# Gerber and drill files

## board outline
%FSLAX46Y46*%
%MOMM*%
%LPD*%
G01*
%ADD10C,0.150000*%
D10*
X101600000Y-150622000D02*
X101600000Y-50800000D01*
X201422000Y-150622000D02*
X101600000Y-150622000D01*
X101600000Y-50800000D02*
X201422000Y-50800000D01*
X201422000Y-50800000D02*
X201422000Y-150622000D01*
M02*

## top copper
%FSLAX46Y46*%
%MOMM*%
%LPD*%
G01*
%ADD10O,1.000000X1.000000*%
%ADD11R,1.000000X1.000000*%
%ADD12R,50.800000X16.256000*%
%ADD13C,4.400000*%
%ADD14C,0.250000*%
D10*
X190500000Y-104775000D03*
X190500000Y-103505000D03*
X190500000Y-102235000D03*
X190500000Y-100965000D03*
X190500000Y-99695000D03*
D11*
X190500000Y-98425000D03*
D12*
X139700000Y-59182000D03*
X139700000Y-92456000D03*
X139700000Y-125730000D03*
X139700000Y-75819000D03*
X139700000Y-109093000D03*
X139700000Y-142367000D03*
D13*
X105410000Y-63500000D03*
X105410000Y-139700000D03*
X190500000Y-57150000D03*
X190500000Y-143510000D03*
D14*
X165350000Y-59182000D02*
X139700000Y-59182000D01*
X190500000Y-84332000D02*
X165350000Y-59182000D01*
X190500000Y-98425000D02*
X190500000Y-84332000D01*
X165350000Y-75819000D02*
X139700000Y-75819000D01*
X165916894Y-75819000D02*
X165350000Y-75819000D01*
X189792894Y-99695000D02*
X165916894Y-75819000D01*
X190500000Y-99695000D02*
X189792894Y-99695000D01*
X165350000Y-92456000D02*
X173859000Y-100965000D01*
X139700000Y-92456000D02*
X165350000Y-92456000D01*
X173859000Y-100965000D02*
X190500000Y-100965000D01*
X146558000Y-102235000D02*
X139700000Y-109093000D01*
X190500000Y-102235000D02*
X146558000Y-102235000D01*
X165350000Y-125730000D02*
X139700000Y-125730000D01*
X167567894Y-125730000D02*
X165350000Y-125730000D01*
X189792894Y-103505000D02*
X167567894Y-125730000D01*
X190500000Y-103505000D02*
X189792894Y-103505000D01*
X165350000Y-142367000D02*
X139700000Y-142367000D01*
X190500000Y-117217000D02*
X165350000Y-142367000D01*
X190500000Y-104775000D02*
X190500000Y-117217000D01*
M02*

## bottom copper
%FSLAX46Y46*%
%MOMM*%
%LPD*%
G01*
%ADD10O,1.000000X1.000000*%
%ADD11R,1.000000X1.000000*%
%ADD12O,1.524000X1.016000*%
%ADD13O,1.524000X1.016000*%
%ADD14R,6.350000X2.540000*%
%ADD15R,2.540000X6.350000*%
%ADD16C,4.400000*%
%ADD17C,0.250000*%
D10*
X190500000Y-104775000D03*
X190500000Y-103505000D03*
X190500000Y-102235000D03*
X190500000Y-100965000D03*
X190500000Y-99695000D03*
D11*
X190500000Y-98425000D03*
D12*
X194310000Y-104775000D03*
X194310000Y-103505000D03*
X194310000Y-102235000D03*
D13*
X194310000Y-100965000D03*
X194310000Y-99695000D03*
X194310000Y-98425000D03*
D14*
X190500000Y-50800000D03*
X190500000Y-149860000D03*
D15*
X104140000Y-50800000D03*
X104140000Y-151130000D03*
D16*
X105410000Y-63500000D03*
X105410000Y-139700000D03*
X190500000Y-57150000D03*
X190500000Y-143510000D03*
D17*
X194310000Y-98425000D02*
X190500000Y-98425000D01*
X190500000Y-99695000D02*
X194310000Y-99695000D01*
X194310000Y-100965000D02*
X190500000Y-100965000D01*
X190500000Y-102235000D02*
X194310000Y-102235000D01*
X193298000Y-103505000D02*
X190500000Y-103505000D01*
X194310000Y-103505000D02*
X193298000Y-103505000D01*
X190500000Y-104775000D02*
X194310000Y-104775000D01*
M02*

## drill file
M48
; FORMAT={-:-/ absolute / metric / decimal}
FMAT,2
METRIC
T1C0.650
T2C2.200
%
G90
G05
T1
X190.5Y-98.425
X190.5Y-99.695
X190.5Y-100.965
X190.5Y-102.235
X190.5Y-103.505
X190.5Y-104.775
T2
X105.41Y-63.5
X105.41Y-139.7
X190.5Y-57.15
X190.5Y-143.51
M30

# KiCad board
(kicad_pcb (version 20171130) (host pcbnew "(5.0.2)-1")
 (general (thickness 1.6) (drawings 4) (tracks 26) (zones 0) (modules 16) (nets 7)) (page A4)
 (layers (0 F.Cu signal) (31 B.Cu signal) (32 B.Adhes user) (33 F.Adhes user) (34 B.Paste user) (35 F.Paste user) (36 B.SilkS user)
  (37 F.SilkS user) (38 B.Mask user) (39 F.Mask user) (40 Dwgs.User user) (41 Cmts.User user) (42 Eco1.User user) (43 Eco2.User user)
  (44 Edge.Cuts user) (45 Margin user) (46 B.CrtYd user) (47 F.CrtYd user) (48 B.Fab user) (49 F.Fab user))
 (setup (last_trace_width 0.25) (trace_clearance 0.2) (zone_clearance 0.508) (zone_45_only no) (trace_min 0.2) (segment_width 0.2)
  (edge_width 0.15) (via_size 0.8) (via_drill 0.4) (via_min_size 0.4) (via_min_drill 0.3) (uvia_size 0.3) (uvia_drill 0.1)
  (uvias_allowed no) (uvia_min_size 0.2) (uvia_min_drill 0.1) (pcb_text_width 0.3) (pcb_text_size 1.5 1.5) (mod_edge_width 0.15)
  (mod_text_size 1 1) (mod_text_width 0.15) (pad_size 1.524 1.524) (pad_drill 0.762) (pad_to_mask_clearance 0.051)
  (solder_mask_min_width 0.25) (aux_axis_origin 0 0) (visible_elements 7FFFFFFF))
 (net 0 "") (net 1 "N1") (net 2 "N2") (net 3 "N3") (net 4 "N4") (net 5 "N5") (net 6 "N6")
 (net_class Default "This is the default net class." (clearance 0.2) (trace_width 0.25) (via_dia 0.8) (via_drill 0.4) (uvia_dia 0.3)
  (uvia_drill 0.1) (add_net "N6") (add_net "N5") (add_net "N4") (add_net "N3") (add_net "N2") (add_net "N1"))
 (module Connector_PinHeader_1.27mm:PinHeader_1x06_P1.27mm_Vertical (layer F.Cu) (at 190.5 98.425)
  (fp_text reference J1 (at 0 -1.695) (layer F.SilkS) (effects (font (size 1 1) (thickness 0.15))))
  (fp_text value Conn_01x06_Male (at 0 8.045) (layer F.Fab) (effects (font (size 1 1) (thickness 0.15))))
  (pad 6 thru_hole oval (at 0 6.35) (size 1 1) (drill 0.65) (layers *.Cu *.Mask) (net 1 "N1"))
  (pad 5 thru_hole oval (at 0 5.08) (size 1 1) (drill 0.65) (layers *.Cu *.Mask) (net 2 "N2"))
  (pad 4 thru_hole oval (at 0 3.81) (size 1 1) (drill 0.65) (layers *.Cu *.Mask) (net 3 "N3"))
  (pad 3 thru_hole oval (at 0 2.54) (size 1 1) (drill 0.65) (layers *.Cu *.Mask) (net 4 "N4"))
  (pad 2 thru_hole oval (at 0 1.27) (size 1 1) (drill 0.65) (layers *.Cu *.Mask) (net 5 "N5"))
  (pad 1 thru_hole rect (at 0 0) (size 1 1) (drill 0.65) (layers *.Cu *.Mask) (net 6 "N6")))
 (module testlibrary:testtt (layer B.Cu) (at 194.31 95.885 180)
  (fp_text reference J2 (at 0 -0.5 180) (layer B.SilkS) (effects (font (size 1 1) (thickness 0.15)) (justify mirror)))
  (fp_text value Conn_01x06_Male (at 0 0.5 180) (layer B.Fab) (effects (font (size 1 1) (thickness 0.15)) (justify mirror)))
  (pad 6 smd oval (at 0 -8.89 180) (size 1.524 1.016) (layers B.Cu B.Paste B.Mask) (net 1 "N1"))
  (pad 5 smd oval (at 0 -7.62 180) (size 1.524 1.016) (layers B.Cu B.Paste B.Mask) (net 2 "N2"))
  (pad 4 smd oval (at 0 -6.35 180) (size 1.524 1.016) (layers B.Cu B.Paste B.Mask) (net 3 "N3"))
  (pad 3 connect oval (at 0 -5.08 180) (size 1.524 1.016) (layers B.Cu B.Mask) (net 4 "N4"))
  (pad 2 connect oval (at 0 -3.81 180) (size 1.524 1.016) (layers B.Cu B.Mask) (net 5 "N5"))
  (pad 1 connect oval (at 0 -2.54 180) (size 1.524 1.016) (layers B.Cu B.Mask) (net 6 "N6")))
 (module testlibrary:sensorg (layer F.Cu) (at 154.94 49.022)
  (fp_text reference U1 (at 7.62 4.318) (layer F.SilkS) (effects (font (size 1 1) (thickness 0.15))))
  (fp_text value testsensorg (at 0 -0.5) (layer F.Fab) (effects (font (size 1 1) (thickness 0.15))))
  (pad 1 connect rect (at -15.24 10.16) (size 50.8 16.256) (layers F.Cu) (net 6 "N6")))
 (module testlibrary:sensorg (layer F.Cu) (at 154.94 82.296)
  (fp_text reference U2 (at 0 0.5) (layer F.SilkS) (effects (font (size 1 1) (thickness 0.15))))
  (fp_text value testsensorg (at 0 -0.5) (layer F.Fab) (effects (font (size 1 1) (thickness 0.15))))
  (pad 1 connect rect (at -15.24 10.16) (size 50.8 16.256) (layers F.Cu) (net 4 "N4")))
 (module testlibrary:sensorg (layer F.Cu) (at 154.94 115.57)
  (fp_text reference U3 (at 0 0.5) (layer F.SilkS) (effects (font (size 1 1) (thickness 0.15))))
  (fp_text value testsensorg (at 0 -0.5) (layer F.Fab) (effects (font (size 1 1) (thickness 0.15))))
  (pad 1 connect rect (at -15.24 10.16) (size 50.8 16.256) (layers F.Cu) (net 2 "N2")))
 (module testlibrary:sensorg (layer F.Cu) (at 154.94 65.659)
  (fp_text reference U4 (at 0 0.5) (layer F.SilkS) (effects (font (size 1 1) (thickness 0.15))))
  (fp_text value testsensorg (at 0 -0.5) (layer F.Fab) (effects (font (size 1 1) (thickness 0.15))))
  (pad 1 connect rect (at -15.24 10.16) (size 50.8 16.256) (layers F.Cu) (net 5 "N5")))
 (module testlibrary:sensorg (layer F.Cu) (at 154.94 98.933)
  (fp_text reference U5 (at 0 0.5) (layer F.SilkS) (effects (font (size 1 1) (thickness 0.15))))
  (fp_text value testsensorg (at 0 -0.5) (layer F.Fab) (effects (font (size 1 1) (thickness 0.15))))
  (pad 1 connect rect (at -15.24 10.16) (size 50.8 16.256) (layers F.Cu) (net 3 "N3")))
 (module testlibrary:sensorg (layer F.Cu) (at 154.94 132.207)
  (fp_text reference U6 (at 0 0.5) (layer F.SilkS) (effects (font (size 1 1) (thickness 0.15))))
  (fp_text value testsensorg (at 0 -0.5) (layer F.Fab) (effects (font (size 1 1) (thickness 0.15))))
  (pad 1 connect rect (at -15.24 10.16) (size 50.8 16.256) (layers F.Cu) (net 1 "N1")))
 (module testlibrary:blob (layer B.Cu) (at 190.5 53.34)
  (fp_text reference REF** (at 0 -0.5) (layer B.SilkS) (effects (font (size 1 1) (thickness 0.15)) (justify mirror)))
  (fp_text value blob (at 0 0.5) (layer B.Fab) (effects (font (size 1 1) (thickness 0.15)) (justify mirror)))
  (pad 1 connect rect (at 0 -2.54) (size 6.35 2.54) (layers B.Cu B.Mask)))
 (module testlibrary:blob (layer B.Cu) (at 190.5 152.4)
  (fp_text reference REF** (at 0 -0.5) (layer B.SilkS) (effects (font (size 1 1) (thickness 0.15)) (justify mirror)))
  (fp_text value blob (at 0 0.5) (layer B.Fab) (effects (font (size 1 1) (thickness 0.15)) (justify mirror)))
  (pad 1 connect rect (at 0 -2.54) (size 6.35 2.54) (layers B.Cu B.Mask)))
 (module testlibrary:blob (layer B.Cu) (at 101.6 50.8 270)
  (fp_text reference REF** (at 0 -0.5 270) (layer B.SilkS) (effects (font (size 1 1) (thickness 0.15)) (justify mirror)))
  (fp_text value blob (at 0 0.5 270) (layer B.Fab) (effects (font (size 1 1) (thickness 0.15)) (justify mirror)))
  (pad 1 connect rect (at 0 -2.54 270) (size 6.35 2.54) (layers B.Cu B.Mask)))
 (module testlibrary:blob (layer B.Cu) (at 101.6 151.13 270)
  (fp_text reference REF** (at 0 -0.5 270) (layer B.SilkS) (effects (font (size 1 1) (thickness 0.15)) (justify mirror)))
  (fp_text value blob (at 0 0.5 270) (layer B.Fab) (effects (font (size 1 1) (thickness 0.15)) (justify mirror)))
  (pad 1 connect rect (at 0 -2.54 270) (size 6.35 2.54) (layers B.Cu B.Mask)))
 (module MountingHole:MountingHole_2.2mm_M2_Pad (layer F.Cu) (at 105.41 63.5)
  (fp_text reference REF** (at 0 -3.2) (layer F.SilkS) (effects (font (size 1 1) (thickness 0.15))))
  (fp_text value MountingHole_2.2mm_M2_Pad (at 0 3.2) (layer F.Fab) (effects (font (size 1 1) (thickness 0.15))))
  (pad 1 thru_hole circle (at 0 0) (size 4.4 4.4) (drill 2.2) (layers *.Cu *.Mask)))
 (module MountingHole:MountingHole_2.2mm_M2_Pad (layer F.Cu) (at 105.41 139.7)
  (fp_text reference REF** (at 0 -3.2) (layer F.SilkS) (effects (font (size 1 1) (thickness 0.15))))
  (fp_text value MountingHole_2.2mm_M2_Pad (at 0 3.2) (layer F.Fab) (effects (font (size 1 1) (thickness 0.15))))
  (pad 1 thru_hole circle (at 0 0) (size 4.4 4.4) (drill 2.2) (layers *.Cu *.Mask)))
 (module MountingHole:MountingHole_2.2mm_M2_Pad (layer F.Cu) (at 190.5 57.15)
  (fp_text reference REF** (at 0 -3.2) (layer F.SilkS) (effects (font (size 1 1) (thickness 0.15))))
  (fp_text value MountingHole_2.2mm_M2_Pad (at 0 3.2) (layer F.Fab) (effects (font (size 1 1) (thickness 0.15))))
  (pad 1 thru_hole circle (at 0 0) (size 4.4 4.4) (drill 2.2) (layers *.Cu *.Mask)))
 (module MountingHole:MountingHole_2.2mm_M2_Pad (layer F.Cu) (at 190.5 143.51)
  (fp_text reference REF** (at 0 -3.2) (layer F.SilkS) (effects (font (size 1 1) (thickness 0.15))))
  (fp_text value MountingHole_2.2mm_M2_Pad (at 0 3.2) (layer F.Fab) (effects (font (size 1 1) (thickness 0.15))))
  (pad 1 thru_hole circle (at 0 0) (size 4.4 4.4) (drill 2.2) (layers *.Cu *.Mask)))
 (gr_line (start 101.6 150.622) (end 101.6 50.8) (layer Edge.Cuts) (width 0.15))
 (gr_line (start 201.422 150.622) (end 101.6 150.622) (layer Edge.Cuts) (width 0.15))
 (gr_line (start 101.6 50.8) (end 201.422 50.8) (layer Edge.Cuts) (width 0.15))
 (gr_line (start 201.422 50.8) (end 201.422 150.622) (layer Edge.Cuts) (width 0.15))
 (segment (start 194.31 98.425) (end 190.5 98.425) (width 0.25) (layer B.Cu) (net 6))
 (segment (start 165.35 59.182) (end 139.7 59.182) (width 0.25) (layer F.Cu) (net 6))
 (segment (start 190.5 84.332) (end 165.35 59.182) (width 0.25) (layer F.Cu) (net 6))
 (segment (start 190.5 98.425) (end 190.5 84.332) (width 0.25) (layer F.Cu) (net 6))
 (segment (start 190.5 99.695) (end 194.31 99.695) (width 0.25) (layer B.Cu) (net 5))
 (segment (start 165.35 75.819) (end 139.7 75.819) (width 0.25) (layer F.Cu) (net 5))
 (segment (start 165.916894 75.819) (end 165.35 75.819) (width 0.25) (layer F.Cu) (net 5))
 (segment (start 189.792894 99.695) (end 165.916894 75.819) (width 0.25) (layer F.Cu) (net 5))
 (segment (start 190.5 99.695) (end 189.792894 99.695) (width 0.25) (layer F.Cu) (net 5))
 (segment (start 194.31 100.965) (end 190.5 100.965) (width 0.25) (layer B.Cu) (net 4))
 (segment (start 165.35 92.456) (end 173.859 100.965) (width 0.25) (layer F.Cu) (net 4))
 (segment (start 139.7 92.456) (end 165.35 92.456) (width 0.25) (layer F.Cu) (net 4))
 (segment (start 173.859 100.965) (end 190.5 100.965) (width 0.25) (layer F.Cu) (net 4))
 (segment (start 190.5 102.235) (end 194.31 102.235) (width 0.25) (layer B.Cu) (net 3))
 (segment (start 146.558 102.235) (end 139.7 109.093) (width 0.25) (layer F.Cu) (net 3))
 (segment (start 190.5 102.235) (end 146.558 102.235) (width 0.25) (layer F.Cu) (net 3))
 (segment (start 193.298 103.505) (end 190.5 103.505) (width 0.25) (layer B.Cu) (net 2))
 (segment (start 194.31 103.505) (end 193.298 103.505) (width 0.25) (layer B.Cu) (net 2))
 (segment (start 165.35 125.73) (end 139.7 125.73) (width 0.25) (layer F.Cu) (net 2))
 (segment (start 167.567894 125.73) (end 165.35 125.73) (width 0.25) (layer F.Cu) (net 2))
 (segment (start 189.792894 103.505) (end 167.567894 125.73) (width 0.25) (layer F.Cu) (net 2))
 (segment (start 190.5 103.505) (end 189.792894 103.505) (width 0.25) (layer F.Cu) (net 2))
 (segment (start 190.5 104.775) (end 194.31 104.775) (width 0.25) (layer B.Cu) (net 1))
 (segment (start 165.35 142.367) (end 139.7 142.367) (width 0.25) (layer F.Cu) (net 1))
 (segment (start 190.5 117.217) (end 165.35 142.367) (width 0.25) (layer F.Cu) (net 1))
 (segment (start 190.5 104.775) (end 190.5 117.217) (width 0.25) (layer F.Cu) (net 1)))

